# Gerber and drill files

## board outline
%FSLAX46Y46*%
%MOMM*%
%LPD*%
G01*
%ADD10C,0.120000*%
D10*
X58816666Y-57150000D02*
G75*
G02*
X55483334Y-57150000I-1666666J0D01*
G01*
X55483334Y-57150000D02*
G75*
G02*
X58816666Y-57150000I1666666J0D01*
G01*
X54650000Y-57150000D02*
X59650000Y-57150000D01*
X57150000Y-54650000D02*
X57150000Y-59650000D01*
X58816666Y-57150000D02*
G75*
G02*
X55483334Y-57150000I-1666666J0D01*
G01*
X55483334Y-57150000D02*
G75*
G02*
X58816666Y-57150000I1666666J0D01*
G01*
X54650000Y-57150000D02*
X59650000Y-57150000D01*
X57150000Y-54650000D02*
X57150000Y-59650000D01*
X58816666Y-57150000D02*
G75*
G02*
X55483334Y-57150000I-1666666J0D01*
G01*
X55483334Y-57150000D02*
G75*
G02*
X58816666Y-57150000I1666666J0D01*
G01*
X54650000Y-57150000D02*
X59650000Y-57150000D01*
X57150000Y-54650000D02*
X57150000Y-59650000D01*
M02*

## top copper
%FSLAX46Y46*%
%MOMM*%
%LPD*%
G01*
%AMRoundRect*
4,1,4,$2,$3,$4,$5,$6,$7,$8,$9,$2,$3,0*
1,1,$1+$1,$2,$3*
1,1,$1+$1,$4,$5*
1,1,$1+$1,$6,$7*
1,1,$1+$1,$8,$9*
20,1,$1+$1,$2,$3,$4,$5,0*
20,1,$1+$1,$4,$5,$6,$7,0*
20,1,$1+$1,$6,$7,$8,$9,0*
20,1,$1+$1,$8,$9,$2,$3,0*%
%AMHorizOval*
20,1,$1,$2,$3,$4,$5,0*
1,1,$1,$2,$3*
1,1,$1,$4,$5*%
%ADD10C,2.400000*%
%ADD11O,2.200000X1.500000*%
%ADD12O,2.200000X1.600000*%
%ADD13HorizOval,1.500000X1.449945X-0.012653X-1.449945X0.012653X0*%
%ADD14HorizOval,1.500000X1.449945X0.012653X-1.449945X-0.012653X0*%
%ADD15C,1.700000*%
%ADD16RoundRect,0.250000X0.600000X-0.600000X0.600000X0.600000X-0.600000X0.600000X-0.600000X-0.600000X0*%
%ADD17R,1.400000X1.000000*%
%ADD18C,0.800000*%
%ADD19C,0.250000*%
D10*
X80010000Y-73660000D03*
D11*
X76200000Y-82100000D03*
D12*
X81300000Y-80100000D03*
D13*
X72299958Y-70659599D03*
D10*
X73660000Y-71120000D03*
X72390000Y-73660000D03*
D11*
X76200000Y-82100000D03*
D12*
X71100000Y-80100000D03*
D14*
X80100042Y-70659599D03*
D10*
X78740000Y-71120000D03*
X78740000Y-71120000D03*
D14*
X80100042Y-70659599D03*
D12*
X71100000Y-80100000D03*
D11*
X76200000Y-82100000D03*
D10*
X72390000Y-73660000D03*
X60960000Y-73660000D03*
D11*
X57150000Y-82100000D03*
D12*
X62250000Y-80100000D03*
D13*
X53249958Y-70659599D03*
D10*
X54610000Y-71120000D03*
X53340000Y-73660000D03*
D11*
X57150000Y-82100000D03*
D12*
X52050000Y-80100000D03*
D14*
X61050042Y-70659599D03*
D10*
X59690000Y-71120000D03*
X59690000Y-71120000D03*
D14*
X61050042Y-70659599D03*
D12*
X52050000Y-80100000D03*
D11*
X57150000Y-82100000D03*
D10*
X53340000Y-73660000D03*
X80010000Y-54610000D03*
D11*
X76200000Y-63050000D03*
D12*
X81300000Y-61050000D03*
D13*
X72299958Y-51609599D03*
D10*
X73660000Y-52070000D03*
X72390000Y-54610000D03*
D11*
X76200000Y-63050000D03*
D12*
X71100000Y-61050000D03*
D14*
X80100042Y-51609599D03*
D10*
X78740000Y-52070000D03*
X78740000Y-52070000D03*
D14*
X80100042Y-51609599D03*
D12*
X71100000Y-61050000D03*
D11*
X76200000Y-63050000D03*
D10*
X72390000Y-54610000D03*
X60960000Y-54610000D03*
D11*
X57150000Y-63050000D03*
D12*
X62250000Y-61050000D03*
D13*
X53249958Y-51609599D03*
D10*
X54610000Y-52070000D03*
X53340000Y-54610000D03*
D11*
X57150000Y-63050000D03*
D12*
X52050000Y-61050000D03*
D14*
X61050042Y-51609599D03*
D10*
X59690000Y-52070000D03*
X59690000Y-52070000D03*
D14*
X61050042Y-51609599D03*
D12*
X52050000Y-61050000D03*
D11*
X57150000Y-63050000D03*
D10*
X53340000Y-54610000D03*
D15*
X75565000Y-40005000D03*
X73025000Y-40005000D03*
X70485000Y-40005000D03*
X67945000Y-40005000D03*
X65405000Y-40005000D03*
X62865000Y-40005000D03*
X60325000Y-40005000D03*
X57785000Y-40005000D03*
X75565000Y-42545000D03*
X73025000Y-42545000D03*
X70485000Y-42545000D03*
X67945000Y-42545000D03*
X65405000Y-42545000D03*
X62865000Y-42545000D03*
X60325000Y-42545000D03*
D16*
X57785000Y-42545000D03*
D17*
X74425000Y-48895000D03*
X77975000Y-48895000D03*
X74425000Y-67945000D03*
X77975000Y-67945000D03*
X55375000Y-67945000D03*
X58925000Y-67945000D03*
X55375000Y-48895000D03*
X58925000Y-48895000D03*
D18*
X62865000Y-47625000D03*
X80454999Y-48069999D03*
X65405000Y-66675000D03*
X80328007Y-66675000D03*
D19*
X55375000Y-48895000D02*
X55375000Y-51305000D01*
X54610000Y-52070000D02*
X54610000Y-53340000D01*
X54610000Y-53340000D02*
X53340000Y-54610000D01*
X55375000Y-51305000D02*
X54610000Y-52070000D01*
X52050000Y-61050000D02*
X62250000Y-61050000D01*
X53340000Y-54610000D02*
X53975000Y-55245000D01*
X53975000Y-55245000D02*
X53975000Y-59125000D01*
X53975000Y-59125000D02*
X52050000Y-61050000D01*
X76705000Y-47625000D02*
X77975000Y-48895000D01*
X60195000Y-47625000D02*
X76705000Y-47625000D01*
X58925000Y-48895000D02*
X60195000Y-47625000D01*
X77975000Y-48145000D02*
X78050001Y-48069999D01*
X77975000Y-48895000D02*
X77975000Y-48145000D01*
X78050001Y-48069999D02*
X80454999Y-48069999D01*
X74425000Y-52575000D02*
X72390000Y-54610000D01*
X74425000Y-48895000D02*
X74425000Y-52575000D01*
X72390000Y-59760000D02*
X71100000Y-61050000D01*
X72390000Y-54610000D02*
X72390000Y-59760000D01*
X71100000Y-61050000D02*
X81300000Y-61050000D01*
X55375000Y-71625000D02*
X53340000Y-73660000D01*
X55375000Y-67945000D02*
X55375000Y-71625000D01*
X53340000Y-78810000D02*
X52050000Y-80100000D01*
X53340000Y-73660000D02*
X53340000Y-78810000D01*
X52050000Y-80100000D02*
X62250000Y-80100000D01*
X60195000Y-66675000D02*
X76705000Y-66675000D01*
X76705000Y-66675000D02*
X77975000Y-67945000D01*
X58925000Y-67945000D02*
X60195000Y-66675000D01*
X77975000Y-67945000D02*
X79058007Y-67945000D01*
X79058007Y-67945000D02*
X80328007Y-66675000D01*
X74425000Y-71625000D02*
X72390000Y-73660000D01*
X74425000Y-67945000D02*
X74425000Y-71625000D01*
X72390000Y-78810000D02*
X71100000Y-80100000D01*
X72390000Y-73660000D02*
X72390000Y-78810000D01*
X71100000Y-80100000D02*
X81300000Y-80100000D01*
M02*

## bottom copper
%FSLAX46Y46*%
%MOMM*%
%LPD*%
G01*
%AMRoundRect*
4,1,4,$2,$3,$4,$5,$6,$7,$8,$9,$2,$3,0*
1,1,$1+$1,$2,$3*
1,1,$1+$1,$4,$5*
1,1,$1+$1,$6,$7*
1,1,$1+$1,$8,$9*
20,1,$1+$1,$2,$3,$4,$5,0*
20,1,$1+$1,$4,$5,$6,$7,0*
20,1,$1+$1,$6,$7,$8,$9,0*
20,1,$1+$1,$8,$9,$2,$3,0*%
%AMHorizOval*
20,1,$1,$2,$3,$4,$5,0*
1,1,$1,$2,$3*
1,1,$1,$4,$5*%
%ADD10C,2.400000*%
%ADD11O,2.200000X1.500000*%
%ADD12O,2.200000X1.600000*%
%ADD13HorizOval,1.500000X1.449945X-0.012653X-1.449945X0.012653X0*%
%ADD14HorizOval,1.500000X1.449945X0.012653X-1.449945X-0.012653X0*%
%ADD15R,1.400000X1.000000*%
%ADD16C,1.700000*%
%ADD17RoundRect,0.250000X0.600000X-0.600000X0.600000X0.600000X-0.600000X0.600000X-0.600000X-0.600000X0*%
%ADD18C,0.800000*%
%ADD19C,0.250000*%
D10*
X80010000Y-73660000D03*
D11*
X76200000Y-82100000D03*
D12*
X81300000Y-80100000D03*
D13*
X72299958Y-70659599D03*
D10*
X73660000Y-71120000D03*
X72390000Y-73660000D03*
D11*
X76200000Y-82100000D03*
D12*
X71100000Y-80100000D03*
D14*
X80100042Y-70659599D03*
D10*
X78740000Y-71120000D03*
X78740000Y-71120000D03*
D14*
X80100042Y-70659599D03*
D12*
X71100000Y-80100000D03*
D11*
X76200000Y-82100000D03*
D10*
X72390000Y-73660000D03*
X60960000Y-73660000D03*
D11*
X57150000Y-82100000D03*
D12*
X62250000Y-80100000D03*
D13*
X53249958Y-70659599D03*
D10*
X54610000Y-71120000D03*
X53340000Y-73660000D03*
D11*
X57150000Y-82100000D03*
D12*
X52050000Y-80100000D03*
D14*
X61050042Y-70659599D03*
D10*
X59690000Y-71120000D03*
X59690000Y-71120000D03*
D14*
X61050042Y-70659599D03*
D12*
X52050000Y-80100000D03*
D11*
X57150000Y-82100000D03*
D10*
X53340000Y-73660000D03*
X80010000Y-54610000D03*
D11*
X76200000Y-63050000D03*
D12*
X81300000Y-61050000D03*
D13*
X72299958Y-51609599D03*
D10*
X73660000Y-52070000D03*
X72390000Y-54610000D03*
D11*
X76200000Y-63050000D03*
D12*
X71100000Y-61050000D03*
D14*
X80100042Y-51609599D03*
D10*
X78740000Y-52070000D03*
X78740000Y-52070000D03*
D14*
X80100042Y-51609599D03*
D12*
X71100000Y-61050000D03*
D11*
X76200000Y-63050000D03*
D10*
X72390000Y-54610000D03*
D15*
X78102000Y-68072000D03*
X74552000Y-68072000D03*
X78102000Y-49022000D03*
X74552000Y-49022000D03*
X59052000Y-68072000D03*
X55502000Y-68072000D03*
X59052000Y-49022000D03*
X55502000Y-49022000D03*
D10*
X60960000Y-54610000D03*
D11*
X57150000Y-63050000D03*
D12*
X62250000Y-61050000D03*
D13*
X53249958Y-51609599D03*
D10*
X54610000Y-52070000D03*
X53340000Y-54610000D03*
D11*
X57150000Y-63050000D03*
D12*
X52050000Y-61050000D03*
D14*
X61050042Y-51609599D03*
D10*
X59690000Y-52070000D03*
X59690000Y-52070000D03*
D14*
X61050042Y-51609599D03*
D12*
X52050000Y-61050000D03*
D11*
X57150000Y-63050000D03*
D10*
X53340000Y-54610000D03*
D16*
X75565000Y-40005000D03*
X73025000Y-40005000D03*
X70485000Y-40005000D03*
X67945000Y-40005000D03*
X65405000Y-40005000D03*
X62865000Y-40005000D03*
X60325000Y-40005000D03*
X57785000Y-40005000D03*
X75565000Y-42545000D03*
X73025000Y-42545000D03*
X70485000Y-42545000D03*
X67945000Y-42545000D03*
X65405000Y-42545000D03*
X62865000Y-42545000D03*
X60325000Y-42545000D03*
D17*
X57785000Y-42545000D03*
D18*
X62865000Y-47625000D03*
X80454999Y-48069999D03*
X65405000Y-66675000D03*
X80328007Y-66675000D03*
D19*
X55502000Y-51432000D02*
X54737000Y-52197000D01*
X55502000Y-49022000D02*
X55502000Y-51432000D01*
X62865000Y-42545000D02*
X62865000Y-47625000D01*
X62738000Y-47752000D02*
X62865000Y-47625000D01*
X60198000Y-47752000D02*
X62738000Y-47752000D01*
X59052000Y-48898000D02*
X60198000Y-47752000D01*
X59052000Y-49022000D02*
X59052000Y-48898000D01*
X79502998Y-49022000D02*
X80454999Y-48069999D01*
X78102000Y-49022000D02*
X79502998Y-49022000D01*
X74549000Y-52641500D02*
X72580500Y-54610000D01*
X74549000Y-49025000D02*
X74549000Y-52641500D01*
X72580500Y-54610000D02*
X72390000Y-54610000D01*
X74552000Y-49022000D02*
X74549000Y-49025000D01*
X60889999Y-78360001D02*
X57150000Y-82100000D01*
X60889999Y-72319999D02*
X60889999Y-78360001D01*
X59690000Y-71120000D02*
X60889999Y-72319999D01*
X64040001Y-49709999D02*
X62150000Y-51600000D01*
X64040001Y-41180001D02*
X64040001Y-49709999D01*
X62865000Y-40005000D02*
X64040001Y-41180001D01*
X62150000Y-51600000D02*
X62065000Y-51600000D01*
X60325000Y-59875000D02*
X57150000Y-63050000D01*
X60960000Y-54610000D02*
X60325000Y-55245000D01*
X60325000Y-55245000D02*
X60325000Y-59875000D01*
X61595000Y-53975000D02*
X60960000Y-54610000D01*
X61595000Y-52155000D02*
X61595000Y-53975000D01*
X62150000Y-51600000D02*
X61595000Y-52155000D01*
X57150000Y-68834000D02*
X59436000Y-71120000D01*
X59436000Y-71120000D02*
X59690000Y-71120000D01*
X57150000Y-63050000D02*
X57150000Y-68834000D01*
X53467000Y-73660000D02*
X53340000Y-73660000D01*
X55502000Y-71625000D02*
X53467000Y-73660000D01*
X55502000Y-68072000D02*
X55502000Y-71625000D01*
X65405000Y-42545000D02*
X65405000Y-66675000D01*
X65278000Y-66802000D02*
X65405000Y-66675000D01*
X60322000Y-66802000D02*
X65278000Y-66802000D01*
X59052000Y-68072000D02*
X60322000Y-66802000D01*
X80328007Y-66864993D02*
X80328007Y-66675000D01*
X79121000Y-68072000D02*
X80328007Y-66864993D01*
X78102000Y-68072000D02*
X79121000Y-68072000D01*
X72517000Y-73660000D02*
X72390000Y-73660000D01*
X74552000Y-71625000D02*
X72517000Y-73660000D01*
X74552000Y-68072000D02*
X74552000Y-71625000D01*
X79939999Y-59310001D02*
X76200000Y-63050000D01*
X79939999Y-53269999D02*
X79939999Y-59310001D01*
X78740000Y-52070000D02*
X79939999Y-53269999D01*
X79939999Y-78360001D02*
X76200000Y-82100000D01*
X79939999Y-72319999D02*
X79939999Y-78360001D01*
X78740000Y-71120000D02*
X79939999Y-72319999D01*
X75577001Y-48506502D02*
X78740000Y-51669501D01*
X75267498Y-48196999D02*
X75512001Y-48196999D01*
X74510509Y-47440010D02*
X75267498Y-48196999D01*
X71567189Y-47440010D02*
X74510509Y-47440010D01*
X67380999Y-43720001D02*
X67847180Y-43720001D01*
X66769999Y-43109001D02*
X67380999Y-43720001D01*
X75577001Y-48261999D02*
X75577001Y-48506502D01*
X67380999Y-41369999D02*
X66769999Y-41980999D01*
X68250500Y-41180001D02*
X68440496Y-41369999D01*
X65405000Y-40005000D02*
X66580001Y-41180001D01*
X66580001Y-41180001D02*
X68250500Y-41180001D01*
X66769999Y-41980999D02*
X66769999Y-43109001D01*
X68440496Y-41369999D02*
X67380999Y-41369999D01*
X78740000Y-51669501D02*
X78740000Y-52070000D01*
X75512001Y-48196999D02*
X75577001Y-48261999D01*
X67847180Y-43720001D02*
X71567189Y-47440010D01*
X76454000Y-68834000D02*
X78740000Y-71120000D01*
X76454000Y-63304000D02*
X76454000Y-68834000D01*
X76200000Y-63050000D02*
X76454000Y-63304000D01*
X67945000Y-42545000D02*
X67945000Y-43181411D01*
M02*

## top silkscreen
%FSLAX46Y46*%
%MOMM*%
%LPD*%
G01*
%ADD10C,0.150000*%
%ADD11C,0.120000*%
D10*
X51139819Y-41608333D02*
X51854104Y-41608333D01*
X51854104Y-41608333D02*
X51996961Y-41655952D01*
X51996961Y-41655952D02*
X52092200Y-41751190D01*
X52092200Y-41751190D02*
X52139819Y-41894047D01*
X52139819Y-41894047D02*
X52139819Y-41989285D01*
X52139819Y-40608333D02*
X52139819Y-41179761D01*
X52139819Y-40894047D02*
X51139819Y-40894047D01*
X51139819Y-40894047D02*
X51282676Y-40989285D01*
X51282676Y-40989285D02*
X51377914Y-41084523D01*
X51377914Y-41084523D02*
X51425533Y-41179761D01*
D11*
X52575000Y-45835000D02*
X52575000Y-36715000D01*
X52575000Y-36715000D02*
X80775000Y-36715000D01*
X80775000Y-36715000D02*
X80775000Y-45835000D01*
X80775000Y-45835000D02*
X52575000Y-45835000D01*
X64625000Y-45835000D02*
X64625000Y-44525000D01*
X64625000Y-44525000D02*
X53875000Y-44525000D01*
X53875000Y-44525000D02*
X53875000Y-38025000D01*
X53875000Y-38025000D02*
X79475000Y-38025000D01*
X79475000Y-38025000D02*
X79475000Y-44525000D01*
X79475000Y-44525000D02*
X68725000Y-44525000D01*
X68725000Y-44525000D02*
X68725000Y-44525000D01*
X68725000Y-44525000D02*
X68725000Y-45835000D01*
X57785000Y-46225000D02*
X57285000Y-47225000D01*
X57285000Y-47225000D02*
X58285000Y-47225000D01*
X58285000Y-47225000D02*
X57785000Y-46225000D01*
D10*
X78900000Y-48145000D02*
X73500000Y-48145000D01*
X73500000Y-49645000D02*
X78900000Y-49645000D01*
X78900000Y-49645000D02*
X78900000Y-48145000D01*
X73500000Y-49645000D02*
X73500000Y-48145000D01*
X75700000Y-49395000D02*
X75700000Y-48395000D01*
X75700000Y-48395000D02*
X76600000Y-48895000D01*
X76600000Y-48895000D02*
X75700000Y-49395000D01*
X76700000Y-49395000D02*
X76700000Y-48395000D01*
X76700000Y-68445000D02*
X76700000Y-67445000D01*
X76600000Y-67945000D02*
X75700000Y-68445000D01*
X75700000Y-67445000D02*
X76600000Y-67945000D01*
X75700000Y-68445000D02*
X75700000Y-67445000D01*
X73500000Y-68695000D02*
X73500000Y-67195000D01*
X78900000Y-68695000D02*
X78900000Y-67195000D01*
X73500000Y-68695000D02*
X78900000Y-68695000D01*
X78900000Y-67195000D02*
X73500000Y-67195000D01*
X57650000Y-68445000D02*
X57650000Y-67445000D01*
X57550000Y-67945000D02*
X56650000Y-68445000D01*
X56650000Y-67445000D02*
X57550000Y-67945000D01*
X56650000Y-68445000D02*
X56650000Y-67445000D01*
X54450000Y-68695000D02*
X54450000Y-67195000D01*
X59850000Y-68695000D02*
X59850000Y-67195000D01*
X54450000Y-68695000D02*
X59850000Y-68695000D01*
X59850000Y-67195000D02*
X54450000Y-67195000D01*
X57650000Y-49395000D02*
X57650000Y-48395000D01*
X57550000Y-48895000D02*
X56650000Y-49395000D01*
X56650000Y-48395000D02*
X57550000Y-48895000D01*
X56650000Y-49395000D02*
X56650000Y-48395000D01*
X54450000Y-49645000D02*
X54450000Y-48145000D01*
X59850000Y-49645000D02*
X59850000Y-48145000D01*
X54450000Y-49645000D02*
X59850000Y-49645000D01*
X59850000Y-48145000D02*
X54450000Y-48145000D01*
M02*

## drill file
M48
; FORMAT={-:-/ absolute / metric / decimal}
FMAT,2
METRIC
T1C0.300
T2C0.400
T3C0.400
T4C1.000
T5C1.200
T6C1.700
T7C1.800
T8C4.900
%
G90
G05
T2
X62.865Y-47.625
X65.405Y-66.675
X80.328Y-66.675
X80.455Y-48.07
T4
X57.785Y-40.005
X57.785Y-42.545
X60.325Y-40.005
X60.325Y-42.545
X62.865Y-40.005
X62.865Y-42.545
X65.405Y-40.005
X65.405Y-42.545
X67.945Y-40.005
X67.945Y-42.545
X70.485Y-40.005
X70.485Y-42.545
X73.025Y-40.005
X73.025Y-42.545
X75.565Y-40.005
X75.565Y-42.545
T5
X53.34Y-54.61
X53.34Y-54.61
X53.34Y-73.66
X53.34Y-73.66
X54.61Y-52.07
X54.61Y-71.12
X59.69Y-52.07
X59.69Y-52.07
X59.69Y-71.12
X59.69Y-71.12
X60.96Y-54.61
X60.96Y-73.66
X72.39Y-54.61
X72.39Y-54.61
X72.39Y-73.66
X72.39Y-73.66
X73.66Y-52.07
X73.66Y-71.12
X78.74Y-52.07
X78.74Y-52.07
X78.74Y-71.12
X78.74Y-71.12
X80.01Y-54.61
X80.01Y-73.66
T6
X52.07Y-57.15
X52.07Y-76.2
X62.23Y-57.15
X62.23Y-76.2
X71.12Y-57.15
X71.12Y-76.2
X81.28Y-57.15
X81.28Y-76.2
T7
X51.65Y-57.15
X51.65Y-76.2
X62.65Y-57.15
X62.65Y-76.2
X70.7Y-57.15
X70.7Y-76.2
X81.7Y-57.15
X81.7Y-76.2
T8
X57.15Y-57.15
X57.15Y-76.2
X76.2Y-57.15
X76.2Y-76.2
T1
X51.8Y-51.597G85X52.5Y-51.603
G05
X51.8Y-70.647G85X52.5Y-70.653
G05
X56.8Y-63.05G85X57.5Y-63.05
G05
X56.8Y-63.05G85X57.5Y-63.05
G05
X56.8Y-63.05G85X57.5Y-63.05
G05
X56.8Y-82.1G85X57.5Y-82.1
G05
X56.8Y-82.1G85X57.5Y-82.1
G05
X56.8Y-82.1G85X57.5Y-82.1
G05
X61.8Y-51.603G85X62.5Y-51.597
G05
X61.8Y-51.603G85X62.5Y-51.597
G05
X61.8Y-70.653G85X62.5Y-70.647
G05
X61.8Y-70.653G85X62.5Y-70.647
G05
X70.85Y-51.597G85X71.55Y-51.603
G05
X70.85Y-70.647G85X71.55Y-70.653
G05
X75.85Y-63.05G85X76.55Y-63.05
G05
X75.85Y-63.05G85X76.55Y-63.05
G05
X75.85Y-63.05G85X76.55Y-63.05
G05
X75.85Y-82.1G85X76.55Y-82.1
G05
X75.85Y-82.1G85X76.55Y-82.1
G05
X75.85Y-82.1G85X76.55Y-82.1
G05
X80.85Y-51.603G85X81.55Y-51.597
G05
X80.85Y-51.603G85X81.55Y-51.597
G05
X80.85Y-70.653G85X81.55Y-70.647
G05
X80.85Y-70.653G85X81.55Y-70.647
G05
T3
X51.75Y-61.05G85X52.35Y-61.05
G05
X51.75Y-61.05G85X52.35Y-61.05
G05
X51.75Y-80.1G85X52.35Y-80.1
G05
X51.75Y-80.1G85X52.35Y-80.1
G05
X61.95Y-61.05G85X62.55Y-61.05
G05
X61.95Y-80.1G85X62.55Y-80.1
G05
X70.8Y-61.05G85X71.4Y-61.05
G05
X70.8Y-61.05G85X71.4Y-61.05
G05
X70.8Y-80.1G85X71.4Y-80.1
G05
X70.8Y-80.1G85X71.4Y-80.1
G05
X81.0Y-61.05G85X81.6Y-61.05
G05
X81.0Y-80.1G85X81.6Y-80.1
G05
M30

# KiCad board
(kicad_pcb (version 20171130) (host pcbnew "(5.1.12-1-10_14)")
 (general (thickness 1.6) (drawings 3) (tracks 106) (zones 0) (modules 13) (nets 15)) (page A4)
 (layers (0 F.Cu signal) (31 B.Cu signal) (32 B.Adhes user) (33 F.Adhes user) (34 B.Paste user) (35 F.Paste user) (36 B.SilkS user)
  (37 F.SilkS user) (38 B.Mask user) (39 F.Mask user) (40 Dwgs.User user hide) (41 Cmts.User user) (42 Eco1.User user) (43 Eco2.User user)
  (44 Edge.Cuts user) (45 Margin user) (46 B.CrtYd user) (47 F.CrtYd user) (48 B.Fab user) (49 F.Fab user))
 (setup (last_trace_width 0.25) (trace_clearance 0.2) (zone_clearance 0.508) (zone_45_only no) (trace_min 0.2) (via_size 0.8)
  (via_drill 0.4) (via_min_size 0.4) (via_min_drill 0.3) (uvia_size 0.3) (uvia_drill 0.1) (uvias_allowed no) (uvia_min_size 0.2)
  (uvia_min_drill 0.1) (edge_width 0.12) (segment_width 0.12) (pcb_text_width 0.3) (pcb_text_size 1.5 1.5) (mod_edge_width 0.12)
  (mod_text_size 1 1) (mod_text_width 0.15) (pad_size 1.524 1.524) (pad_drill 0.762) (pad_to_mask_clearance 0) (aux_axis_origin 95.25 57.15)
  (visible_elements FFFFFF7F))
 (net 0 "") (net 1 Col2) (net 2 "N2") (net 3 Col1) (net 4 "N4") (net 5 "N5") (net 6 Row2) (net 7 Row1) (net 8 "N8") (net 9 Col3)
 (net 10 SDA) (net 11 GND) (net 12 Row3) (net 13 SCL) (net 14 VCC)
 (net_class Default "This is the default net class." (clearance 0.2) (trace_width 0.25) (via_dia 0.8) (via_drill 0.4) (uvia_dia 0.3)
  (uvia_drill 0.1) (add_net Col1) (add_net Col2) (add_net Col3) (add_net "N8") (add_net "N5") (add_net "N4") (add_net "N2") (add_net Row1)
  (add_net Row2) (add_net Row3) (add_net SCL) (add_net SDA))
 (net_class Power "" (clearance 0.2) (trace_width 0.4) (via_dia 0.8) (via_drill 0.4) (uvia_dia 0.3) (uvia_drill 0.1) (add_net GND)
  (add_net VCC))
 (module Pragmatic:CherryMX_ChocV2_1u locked (layer F.Cu) (at 76.2 76.2)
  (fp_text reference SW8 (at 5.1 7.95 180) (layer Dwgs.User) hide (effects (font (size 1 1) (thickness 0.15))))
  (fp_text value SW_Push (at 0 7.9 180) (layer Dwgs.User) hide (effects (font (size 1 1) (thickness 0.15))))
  (pad 2 thru_hole circle (at 3.81 -2.54) (size 2.4 2.4) (drill 1.2) (layers *.Cu B.Mask) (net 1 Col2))
  (pad 2 thru_hole oval (at 0 5.9) (size 2.2 1.5) (drill oval 1 0.3) (layers *.Cu B.Mask) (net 1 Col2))
  (pad 1 thru_hole oval (at 5.1 3.9) (size 2.2 1.6) (drill oval 1 0.4) (layers *.Cu B.Mask) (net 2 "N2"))
  (pad 1 thru_hole oval (at -5 -5.55 359.5) (size 4.4 1.5) (drill oval 1 0.3 (offset 1.1 0)) (layers *.Cu B.Mask) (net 2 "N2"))
  (pad 1 thru_hole circle (at -2.54 -5.08) (size 2.4 2.4) (drill 1.2) (layers *.Cu B.Mask) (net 2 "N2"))
  (pad 1 thru_hole circle (at -3.81 -2.54) (size 2.4 2.4) (drill 1.2) (layers *.Cu B.Mask) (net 2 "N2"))
  (pad 2 thru_hole oval (at 0 5.9) (size 2.2 1.5) (drill oval 1 0.3) (layers *.Cu B.Mask) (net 1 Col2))
  (pad 1 thru_hole oval (at -5.1 3.9) (size 2.2 1.6) (drill oval 1 0.4) (layers *.Cu B.Mask) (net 2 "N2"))
  (pad 2 thru_hole oval (at 5 -5.55 0.5) (size 4.4 1.5) (drill oval 1 0.3 (offset -1.1 0)) (layers *.Cu B.Mask) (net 1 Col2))
  (pad 2 thru_hole circle (at 2.54 -5.08) (size 2.4 2.4) (drill 1.2) (layers *.Cu B.Mask) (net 1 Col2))
  (pad 2 thru_hole circle (at 2.54 -5.08) (size 2.4 2.4) (drill 1.2) (layers *.Cu B.Mask) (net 1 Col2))
  (pad 2 thru_hole oval (at 5 -5.55 0.5) (size 4.4 1.5) (drill oval 1 0.3 (offset -1.1 0)) (layers *.Cu B.Mask) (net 1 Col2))
  (pad 1 thru_hole oval (at -5.1 3.9) (size 2.2 1.6) (drill oval 1 0.4) (layers *.Cu B.Mask) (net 2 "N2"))
  (pad "" np_thru_hole circle (at 0 0 90) (size 4.9 4.9) (drill 4.9) (layers *.Cu *.Mask))
  (pad "" np_thru_hole circle (at -5.5 0 90) (size 1.8 1.8) (drill 1.8) (layers *.Cu *.Mask))
  (pad "" np_thru_hole circle (at 5.5 0 90) (size 1.8 1.8) (drill 1.8) (layers *.Cu *.Mask))
  (pad 2 thru_hole oval (at 0 5.9) (size 2.2 1.5) (drill oval 1 0.3) (layers *.Cu B.Mask) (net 1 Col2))
  (pad 1 thru_hole circle (at -3.81 -2.54) (size 2.4 2.4) (drill 1.2) (layers *.Cu B.Mask) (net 2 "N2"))
  (pad "" np_thru_hole circle (at 5.08 0) (size 1.7 1.7) (drill 1.7) (layers *.Cu *.Mask))
  (pad "" np_thru_hole circle (at -5.08 0) (size 1.7 1.7) (drill 1.7) (layers *.Cu *.Mask)))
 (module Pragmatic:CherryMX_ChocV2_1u (layer F.Cu) (at 57.15 76.2)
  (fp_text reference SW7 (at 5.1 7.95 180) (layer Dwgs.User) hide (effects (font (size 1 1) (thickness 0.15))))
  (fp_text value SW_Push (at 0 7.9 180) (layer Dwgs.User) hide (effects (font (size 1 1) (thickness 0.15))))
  (pad 2 thru_hole circle (at 3.81 -2.54) (size 2.4 2.4) (drill 1.2) (layers *.Cu B.Mask) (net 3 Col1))
  (pad 2 thru_hole oval (at 0 5.9) (size 2.2 1.5) (drill oval 1 0.3) (layers *.Cu B.Mask) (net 3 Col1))
  (pad 1 thru_hole oval (at 5.1 3.9) (size 2.2 1.6) (drill oval 1 0.4) (layers *.Cu B.Mask) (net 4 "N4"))
  (pad 1 thru_hole oval (at -5 -5.55 359.5) (size 4.4 1.5) (drill oval 1 0.3 (offset 1.1 0)) (layers *.Cu B.Mask) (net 4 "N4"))
  (pad 1 thru_hole circle (at -2.54 -5.08) (size 2.4 2.4) (drill 1.2) (layers *.Cu B.Mask) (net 4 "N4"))
  (pad 1 thru_hole circle (at -3.81 -2.54) (size 2.4 2.4) (drill 1.2) (layers *.Cu B.Mask) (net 4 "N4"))
  (pad 2 thru_hole oval (at 0 5.9) (size 2.2 1.5) (drill oval 1 0.3) (layers *.Cu B.Mask) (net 3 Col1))
  (pad 1 thru_hole oval (at -5.1 3.9) (size 2.2 1.6) (drill oval 1 0.4) (layers *.Cu B.Mask) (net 4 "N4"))
  (pad 2 thru_hole oval (at 5 -5.55 0.5) (size 4.4 1.5) (drill oval 1 0.3 (offset -1.1 0)) (layers *.Cu B.Mask) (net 3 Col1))
  (pad 2 thru_hole circle (at 2.54 -5.08) (size 2.4 2.4) (drill 1.2) (layers *.Cu B.Mask) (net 3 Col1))
  (pad 2 thru_hole circle (at 2.54 -5.08) (size 2.4 2.4) (drill 1.2) (layers *.Cu B.Mask) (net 3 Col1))
  (pad 2 thru_hole oval (at 5 -5.55 0.5) (size 4.4 1.5) (drill oval 1 0.3 (offset -1.1 0)) (layers *.Cu B.Mask) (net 3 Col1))
  (pad 1 thru_hole oval (at -5.1 3.9) (size 2.2 1.6) (drill oval 1 0.4) (layers *.Cu B.Mask) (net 4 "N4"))
  (pad "" np_thru_hole circle (at 0 0 90) (size 4.9 4.9) (drill 4.9) (layers *.Cu *.Mask))
  (pad "" np_thru_hole circle (at -5.5 0 90) (size 1.8 1.8) (drill 1.8) (layers *.Cu *.Mask))
  (pad "" np_thru_hole circle (at 5.5 0 90) (size 1.8 1.8) (drill 1.8) (layers *.Cu *.Mask))
  (pad 2 thru_hole oval (at 0 5.9) (size 2.2 1.5) (drill oval 1 0.3) (layers *.Cu B.Mask) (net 3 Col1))
  (pad 1 thru_hole circle (at -3.81 -2.54) (size 2.4 2.4) (drill 1.2) (layers *.Cu B.Mask) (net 4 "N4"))
  (pad "" np_thru_hole circle (at 5.08 0) (size 1.7 1.7) (drill 1.7) (layers *.Cu *.Mask))
  (pad "" np_thru_hole circle (at -5.08 0) (size 1.7 1.7) (drill 1.7) (layers *.Cu *.Mask)))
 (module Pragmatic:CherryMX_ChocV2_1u (layer F.Cu) (at 76.2 57.15)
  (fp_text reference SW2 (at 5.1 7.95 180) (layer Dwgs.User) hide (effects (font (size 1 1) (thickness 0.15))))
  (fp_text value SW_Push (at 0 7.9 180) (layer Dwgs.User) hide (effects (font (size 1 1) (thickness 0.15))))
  (pad 2 thru_hole circle (at 3.81 -2.54) (size 2.4 2.4) (drill 1.2) (layers *.Cu B.Mask) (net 1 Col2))
  (pad 2 thru_hole oval (at 0 5.9) (size 2.2 1.5) (drill oval 1 0.3) (layers *.Cu B.Mask) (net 1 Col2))
  (pad 1 thru_hole oval (at 5.1 3.9) (size 2.2 1.6) (drill oval 1 0.4) (layers *.Cu B.Mask) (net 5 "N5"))
  (pad 1 thru_hole oval (at -5 -5.55 359.5) (size 4.4 1.5) (drill oval 1 0.3 (offset 1.1 0)) (layers *.Cu B.Mask) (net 5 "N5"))
  (pad 1 thru_hole circle (at -2.54 -5.08) (size 2.4 2.4) (drill 1.2) (layers *.Cu B.Mask) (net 5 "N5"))
  (pad 1 thru_hole circle (at -3.81 -2.54) (size 2.4 2.4) (drill 1.2) (layers *.Cu B.Mask) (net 5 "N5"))
  (pad 2 thru_hole oval (at 0 5.9) (size 2.2 1.5) (drill oval 1 0.3) (layers *.Cu B.Mask) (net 1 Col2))
  (pad 1 thru_hole oval (at -5.1 3.9) (size 2.2 1.6) (drill oval 1 0.4) (layers *.Cu B.Mask) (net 5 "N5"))
  (pad 2 thru_hole oval (at 5 -5.55 0.5) (size 4.4 1.5) (drill oval 1 0.3 (offset -1.1 0)) (layers *.Cu B.Mask) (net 1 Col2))
  (pad 2 thru_hole circle (at 2.54 -5.08) (size 2.4 2.4) (drill 1.2) (layers *.Cu B.Mask) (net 1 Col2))
  (pad 2 thru_hole circle (at 2.54 -5.08) (size 2.4 2.4) (drill 1.2) (layers *.Cu B.Mask) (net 1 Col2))
  (pad 2 thru_hole oval (at 5 -5.55 0.5) (size 4.4 1.5) (drill oval 1 0.3 (offset -1.1 0)) (layers *.Cu B.Mask) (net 1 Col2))
  (pad 1 thru_hole oval (at -5.1 3.9) (size 2.2 1.6) (drill oval 1 0.4) (layers *.Cu B.Mask) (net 5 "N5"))
  (pad "" np_thru_hole circle (at 0 0 90) (size 4.9 4.9) (drill 4.9) (layers *.Cu *.Mask))
  (pad "" np_thru_hole circle (at -5.5 0 90) (size 1.8 1.8) (drill 1.8) (layers *.Cu *.Mask))
  (pad "" np_thru_hole circle (at 5.5 0 90) (size 1.8 1.8) (drill 1.8) (layers *.Cu *.Mask))
  (pad 2 thru_hole oval (at 0 5.9) (size 2.2 1.5) (drill oval 1 0.3) (layers *.Cu B.Mask) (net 1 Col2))
  (pad 1 thru_hole circle (at -3.81 -2.54) (size 2.4 2.4) (drill 1.2) (layers *.Cu B.Mask) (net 5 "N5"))
  (pad "" np_thru_hole circle (at 5.08 0) (size 1.7 1.7) (drill 1.7) (layers *.Cu *.Mask))
  (pad "" np_thru_hole circle (at -5.08 0) (size 1.7 1.7) (drill 1.7) (layers *.Cu *.Mask)))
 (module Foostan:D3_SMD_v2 (layer B.Cu) (at 76.327 68.072 180) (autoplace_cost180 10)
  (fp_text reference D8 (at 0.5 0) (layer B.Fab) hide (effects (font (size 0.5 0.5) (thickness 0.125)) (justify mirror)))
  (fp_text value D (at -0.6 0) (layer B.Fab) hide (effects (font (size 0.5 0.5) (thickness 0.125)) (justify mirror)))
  (pad 1 smd rect (at -1.775 0 180) (size 1.4 1) (layers B.Cu B.Paste B.Mask) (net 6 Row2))
  (pad 2 smd rect (at 1.775 0 180) (size 1.4 1) (layers B.Cu B.Paste B.Mask) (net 2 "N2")))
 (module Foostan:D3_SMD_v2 (layer B.Cu) (at 76.327 49.022 180) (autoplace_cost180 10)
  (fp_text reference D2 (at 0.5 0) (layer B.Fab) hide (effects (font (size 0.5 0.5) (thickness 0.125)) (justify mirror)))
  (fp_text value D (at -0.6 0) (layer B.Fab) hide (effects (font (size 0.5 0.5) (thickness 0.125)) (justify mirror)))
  (pad 1 smd rect (at -1.775 0 180) (size 1.4 1) (layers B.Cu B.Paste B.Mask) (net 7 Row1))
  (pad 2 smd rect (at 1.775 0 180) (size 1.4 1) (layers B.Cu B.Paste B.Mask) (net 5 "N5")))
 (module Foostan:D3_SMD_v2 (layer B.Cu) (at 57.277 68.072 180) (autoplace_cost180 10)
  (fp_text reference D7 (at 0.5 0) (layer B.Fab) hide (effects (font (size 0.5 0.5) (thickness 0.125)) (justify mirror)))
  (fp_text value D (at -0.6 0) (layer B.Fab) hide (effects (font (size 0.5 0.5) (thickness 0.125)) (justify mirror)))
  (pad 1 smd rect (at -1.775 0 180) (size 1.4 1) (layers B.Cu B.Paste B.Mask) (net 6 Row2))
  (pad 2 smd rect (at 1.775 0 180) (size 1.4 1) (layers B.Cu B.Paste B.Mask) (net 4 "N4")))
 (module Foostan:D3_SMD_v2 (layer B.Cu) (at 57.277 49.022 180) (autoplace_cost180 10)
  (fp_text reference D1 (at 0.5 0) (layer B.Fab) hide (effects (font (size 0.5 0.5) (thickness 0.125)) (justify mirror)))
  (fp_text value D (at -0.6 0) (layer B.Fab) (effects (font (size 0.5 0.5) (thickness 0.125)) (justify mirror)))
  (pad 1 smd rect (at -1.775 0 180) (size 1.4 1) (layers B.Cu B.Paste B.Mask) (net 7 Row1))
  (pad 2 smd rect (at 1.775 0 180) (size 1.4 1) (layers B.Cu B.Paste B.Mask) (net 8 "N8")))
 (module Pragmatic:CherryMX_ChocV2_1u (layer F.Cu) (at 57.15 57.15)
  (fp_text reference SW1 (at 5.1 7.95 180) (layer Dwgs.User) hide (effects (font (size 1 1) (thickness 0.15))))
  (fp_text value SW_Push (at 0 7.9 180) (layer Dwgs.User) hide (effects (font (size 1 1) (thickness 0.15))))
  (pad 2 thru_hole circle (at 3.81 -2.54) (size 2.4 2.4) (drill 1.2) (layers *.Cu B.Mask) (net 3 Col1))
  (pad 2 thru_hole oval (at 0 5.9) (size 2.2 1.5) (drill oval 1 0.3) (layers *.Cu B.Mask) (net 3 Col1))
  (pad 1 thru_hole oval (at 5.1 3.9) (size 2.2 1.6) (drill oval 1 0.4) (layers *.Cu B.Mask) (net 8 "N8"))
  (pad 1 thru_hole oval (at -5 -5.55 359.5) (size 4.4 1.5) (drill oval 1 0.3 (offset 1.1 0)) (layers *.Cu B.Mask) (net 8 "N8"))
  (pad 1 thru_hole circle (at -2.54 -5.08) (size 2.4 2.4) (drill 1.2) (layers *.Cu B.Mask) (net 8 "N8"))
  (pad 1 thru_hole circle (at -3.81 -2.54) (size 2.4 2.4) (drill 1.2) (layers *.Cu B.Mask) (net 8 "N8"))
  (pad 2 thru_hole oval (at 0 5.9) (size 2.2 1.5) (drill oval 1 0.3) (layers *.Cu B.Mask) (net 3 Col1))
  (pad 1 thru_hole oval (at -5.1 3.9) (size 2.2 1.6) (drill oval 1 0.4) (layers *.Cu B.Mask) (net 8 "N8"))
  (pad 2 thru_hole oval (at 5 -5.55 0.5) (size 4.4 1.5) (drill oval 1 0.3 (offset -1.1 0)) (layers *.Cu B.Mask) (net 3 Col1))
  (pad 2 thru_hole circle (at 2.54 -5.08) (size 2.4 2.4) (drill 1.2) (layers *.Cu B.Mask) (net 3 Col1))
  (pad 2 thru_hole circle (at 2.54 -5.08) (size 2.4 2.4) (drill 1.2) (layers *.Cu B.Mask) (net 3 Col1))
  (pad 2 thru_hole oval (at 5 -5.55 0.5) (size 4.4 1.5) (drill oval 1 0.3 (offset -1.1 0)) (layers *.Cu B.Mask) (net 3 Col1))
  (pad 1 thru_hole oval (at -5.1 3.9) (size 2.2 1.6) (drill oval 1 0.4) (layers *.Cu B.Mask) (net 8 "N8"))
  (pad "" np_thru_hole circle (at 0 0 90) (size 4.9 4.9) (drill 4.9) (layers *.Cu *.Mask))
  (pad "" np_thru_hole circle (at -5.5 0 90) (size 1.8 1.8) (drill 1.8) (layers *.Cu *.Mask))
  (pad "" np_thru_hole circle (at 5.5 0 90) (size 1.8 1.8) (drill 1.8) (layers *.Cu *.Mask))
  (pad 2 thru_hole oval (at 0 5.9) (size 2.2 1.5) (drill oval 1 0.3) (layers *.Cu B.Mask) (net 3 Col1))
  (pad 1 thru_hole circle (at -3.81 -2.54) (size 2.4 2.4) (drill 1.2) (layers *.Cu B.Mask) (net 8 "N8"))
  (pad "" np_thru_hole circle (at 5.08 0) (size 1.7 1.7) (drill 1.7) (layers *.Cu *.Mask))
  (pad "" np_thru_hole circle (at -5.08 0) (size 1.7 1.7) (drill 1.7) (layers *.Cu *.Mask)))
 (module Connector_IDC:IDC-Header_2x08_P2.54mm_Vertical (layer F.Cu) (at 57.785 42.545 90)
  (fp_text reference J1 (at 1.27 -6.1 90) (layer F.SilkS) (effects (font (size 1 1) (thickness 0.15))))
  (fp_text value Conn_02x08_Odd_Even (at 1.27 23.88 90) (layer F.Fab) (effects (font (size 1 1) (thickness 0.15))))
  (fp_line (start -3.29 -5.21) (end 5.83 -5.21) (layer F.SilkS) (width 0.12))
  (fp_line (start 5.83 -5.21) (end 5.83 22.99) (layer F.SilkS) (width 0.12))
  (fp_line (start 5.83 22.99) (end -3.29 22.99) (layer F.SilkS) (width 0.12))
  (fp_line (start -3.29 22.99) (end -3.29 -5.21) (layer F.SilkS) (width 0.12))
  (fp_line (start -3.29 6.84) (end -1.98 6.84) (layer F.SilkS) (width 0.12))
  (fp_line (start -1.98 6.84) (end -1.98 -3.91) (layer F.SilkS) (width 0.12))
  (fp_line (start -1.98 -3.91) (end 4.52 -3.91) (layer F.SilkS) (width 0.12))
  (fp_line (start 4.52 -3.91) (end 4.52 21.69) (layer F.SilkS) (width 0.12))
  (fp_line (start 4.52 21.69) (end -1.98 21.69) (layer F.SilkS) (width 0.12))
  (fp_line (start -1.98 21.69) (end -1.98 10.94) (layer F.SilkS) (width 0.12))
  (fp_line (start -1.98 10.94) (end -1.98 10.94) (layer F.SilkS) (width 0.12))
  (fp_line (start -1.98 10.94) (end -3.29 10.94) (layer F.SilkS) (width 0.12))
  (fp_line (start -3.68 0) (end -4.68 -0.5) (layer F.SilkS) (width 0.12))
  (fp_line (start -4.68 -0.5) (end -4.68 0.5) (layer F.SilkS) (width 0.12))
  (fp_line (start -4.68 0.5) (end -3.68 0) (layer F.SilkS) (width 0.12))
  (pad 16 thru_hole circle (at 2.54 17.78 90) (size 1.7 1.7) (drill 1) (layers *.Cu *.Mask))
  (pad 14 thru_hole circle (at 2.54 15.24 90) (size 1.7 1.7) (drill 1) (layers *.Cu *.Mask))
  (pad 12 thru_hole circle (at 2.54 12.7 90) (size 1.7 1.7) (drill 1) (layers *.Cu *.Mask))
  (pad 10 thru_hole circle (at 2.54 10.16 90) (size 1.7 1.7) (drill 1) (layers *.Cu *.Mask) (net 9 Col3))
  (pad 8 thru_hole circle (at 2.54 7.62 90) (size 1.7 1.7) (drill 1) (layers *.Cu *.Mask) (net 1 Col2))
  (pad 6 thru_hole circle (at 2.54 5.08 90) (size 1.7 1.7) (drill 1) (layers *.Cu *.Mask) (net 3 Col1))
  (pad 4 thru_hole circle (at 2.54 2.54 90) (size 1.7 1.7) (drill 1) (layers *.Cu *.Mask) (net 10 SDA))
  (pad 2 thru_hole circle (at 2.54 0 90) (size 1.7 1.7) (drill 1) (layers *.Cu *.Mask) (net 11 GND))
  (pad 15 thru_hole circle (at 0 17.78 90) (size 1.7 1.7) (drill 1) (layers *.Cu *.Mask))
  (pad 13 thru_hole circle (at 0 15.24 90) (size 1.7 1.7) (drill 1) (layers *.Cu *.Mask))
  (pad 11 thru_hole circle (at 0 12.7 90) (size 1.7 1.7) (drill 1) (layers *.Cu *.Mask))
  (pad 9 thru_hole circle (at 0 10.16 90) (size 1.7 1.7) (drill 1) (layers *.Cu *.Mask) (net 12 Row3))
  (pad 7 thru_hole circle (at 0 7.62 90) (size 1.7 1.7) (drill 1) (layers *.Cu *.Mask) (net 6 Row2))
  (pad 5 thru_hole circle (at 0 5.08 90) (size 1.7 1.7) (drill 1) (layers *.Cu *.Mask) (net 7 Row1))
  (pad 3 thru_hole circle (at 0 2.54 90) (size 1.7 1.7) (drill 1) (layers *.Cu *.Mask) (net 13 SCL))
  (pad 1 thru_hole roundrect (at 0 0 90) (size 1.7 1.7) (drill 1) (layers *.Cu *.Mask) (roundrect_rratio 0.147059) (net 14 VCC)))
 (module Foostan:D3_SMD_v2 (layer F.Cu) (at 76.2 48.895 180) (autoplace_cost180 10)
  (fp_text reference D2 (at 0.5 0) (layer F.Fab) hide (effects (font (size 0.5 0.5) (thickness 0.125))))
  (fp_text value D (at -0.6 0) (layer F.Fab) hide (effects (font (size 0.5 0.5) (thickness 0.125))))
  (fp_line (start -2.7 0.75) (end 2.7 0.75) (layer F.SilkS) (width 0.15))
  (fp_line (start 2.7 -0.75) (end -2.7 -0.75) (layer F.SilkS) (width 0.15))
  (fp_line (start -2.7 -0.75) (end -2.7 0.75) (layer F.SilkS) (width 0.15))
  (fp_line (start 2.7 -0.75) (end 2.7 0.75) (layer F.SilkS) (width 0.15))
  (fp_line (start 0.5 -0.5) (end 0.5 0.5) (layer F.SilkS) (width 0.15))
  (fp_line (start 0.5 0.5) (end -0.4 0) (layer F.SilkS) (width 0.15))
  (fp_line (start -0.4 0) (end 0.5 -0.5) (layer F.SilkS) (width 0.15))
  (fp_line (start -0.5 -0.5) (end -0.5 0.5) (layer F.SilkS) (width 0.15))
  (pad 2 smd rect (at 1.775 0 180) (size 1.4 1) (layers F.Cu F.Paste F.Mask) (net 5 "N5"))
  (pad 1 smd rect (at -1.775 0 180) (size 1.4 1) (layers F.Cu F.Paste F.Mask) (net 7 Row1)))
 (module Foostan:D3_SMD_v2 (layer F.Cu) (at 76.2 67.945 180) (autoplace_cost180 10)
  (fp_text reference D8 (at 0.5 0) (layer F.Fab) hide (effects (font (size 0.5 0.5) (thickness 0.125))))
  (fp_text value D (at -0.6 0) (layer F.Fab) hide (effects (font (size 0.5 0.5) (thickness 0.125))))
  (fp_line (start -0.5 -0.5) (end -0.5 0.5) (layer F.SilkS) (width 0.15))
  (fp_line (start -0.4 0) (end 0.5 -0.5) (layer F.SilkS) (width 0.15))
  (fp_line (start 0.5 0.5) (end -0.4 0) (layer F.SilkS) (width 0.15))
  (fp_line (start 0.5 -0.5) (end 0.5 0.5) (layer F.SilkS) (width 0.15))
  (fp_line (start 2.7 -0.75) (end 2.7 0.75) (layer F.SilkS) (width 0.15))
  (fp_line (start -2.7 -0.75) (end -2.7 0.75) (layer F.SilkS) (width 0.15))
  (fp_line (start 2.7 -0.75) (end -2.7 -0.75) (layer F.SilkS) (width 0.15))
  (fp_line (start -2.7 0.75) (end 2.7 0.75) (layer F.SilkS) (width 0.15))
  (pad 2 smd rect (at 1.775 0 180) (size 1.4 1) (layers F.Cu F.Paste F.Mask) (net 2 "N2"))
  (pad 1 smd rect (at -1.775 0 180) (size 1.4 1) (layers F.Cu F.Paste F.Mask) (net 6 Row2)))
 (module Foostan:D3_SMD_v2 (layer F.Cu) (at 57.15 67.945 180) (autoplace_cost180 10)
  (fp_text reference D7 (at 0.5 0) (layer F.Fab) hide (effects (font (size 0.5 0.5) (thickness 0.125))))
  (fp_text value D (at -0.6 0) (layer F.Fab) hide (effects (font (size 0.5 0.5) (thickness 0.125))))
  (fp_line (start -0.5 -0.5) (end -0.5 0.5) (layer F.SilkS) (width 0.15))
  (fp_line (start -0.4 0) (end 0.5 -0.5) (layer F.SilkS) (width 0.15))
  (fp_line (start 0.5 0.5) (end -0.4 0) (layer F.SilkS) (width 0.15))
  (fp_line (start 0.5 -0.5) (end 0.5 0.5) (layer F.SilkS) (width 0.15))
  (fp_line (start 2.7 -0.75) (end 2.7 0.75) (layer F.SilkS) (width 0.15))
  (fp_line (start -2.7 -0.75) (end -2.7 0.75) (layer F.SilkS) (width 0.15))
  (fp_line (start 2.7 -0.75) (end -2.7 -0.75) (layer F.SilkS) (width 0.15))
  (fp_line (start -2.7 0.75) (end 2.7 0.75) (layer F.SilkS) (width 0.15))
  (pad 2 smd rect (at 1.775 0 180) (size 1.4 1) (layers F.Cu F.Paste F.Mask) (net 4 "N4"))
  (pad 1 smd rect (at -1.775 0 180) (size 1.4 1) (layers F.Cu F.Paste F.Mask) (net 6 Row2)))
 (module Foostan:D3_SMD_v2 (layer F.Cu) (at 57.15 48.895 180) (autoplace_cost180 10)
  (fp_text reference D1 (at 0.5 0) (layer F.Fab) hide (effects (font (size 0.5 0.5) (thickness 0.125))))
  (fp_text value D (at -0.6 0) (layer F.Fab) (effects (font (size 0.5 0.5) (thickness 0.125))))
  (fp_line (start -0.5 -0.5) (end -0.5 0.5) (layer F.SilkS) (width 0.15))
  (fp_line (start -0.4 0) (end 0.5 -0.5) (layer F.SilkS) (width 0.15))
  (fp_line (start 0.5 0.5) (end -0.4 0) (layer F.SilkS) (width 0.15))
  (fp_line (start 0.5 -0.5) (end 0.5 0.5) (layer F.SilkS) (width 0.15))
  (fp_line (start 2.7 -0.75) (end 2.7 0.75) (layer F.SilkS) (width 0.15))
  (fp_line (start -2.7 -0.75) (end -2.7 0.75) (layer F.SilkS) (width 0.15))
  (fp_line (start 2.7 -0.75) (end -2.7 -0.75) (layer F.SilkS) (width 0.15))
  (fp_line (start -2.7 0.75) (end 2.7 0.75) (layer F.SilkS) (width 0.15))
  (pad 2 smd rect (at 1.775 0 180) (size 1.4 1) (layers F.Cu F.Paste F.Mask) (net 8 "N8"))
  (pad 1 smd rect (at -1.775 0 180) (size 1.4 1) (layers F.Cu F.Paste F.Mask) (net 7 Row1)))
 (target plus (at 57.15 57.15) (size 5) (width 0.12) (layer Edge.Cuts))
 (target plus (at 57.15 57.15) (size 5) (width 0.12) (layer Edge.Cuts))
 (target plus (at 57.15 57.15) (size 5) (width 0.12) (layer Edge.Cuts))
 (segment (start 55.375 48.895) (end 55.375 51.305) (width 0.25) (layer F.Cu) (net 8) (status 30))
 (segment (start 54.61 52.07) (end 54.61 53.34) (width 0.25) (layer F.Cu) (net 8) (status 10))
 (segment (start 54.61 53.34) (end 53.34 54.61) (width 0.25) (layer F.Cu) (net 8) (status 20))
 (segment (start 55.375 51.305) (end 54.61 52.07) (width 0.25) (layer F.Cu) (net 8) (status 30))
 (segment (start 52.05 61.05) (end 62.25 61.05) (width 0.25) (layer F.Cu) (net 8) (status 30))
 (segment (start 53.34 54.61) (end 53.975 55.245) (width 0.25) (layer F.Cu) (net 8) (status 30))
 (segment (start 53.975 55.245) (end 53.975 59.125) (width 0.25) (layer F.Cu) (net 8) (status 10))
 (segment (start 53.975 59.125) (end 52.05 61.05) (width 0.25) (layer F.Cu) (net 8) (status 20))
 (segment (start 55.502 51.432) (end 54.737 52.197) (width 0.25) (layer B.Cu) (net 8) (status 30))
 (segment (start 55.502 49.022) (end 55.502 51.432) (width 0.25) (layer B.Cu) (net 8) (status 30))
 (segment (start 76.705 47.625) (end 77.975 48.895) (width 0.25) (layer F.Cu) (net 7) (status 20))
 (segment (start 60.195 47.625) (end 76.705 47.625) (width 0.25) (layer F.Cu) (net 7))
 (segment (start 58.925 48.895) (end 60.195 47.625) (width 0.25) (layer F.Cu) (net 7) (status 10))
 (via (at 62.865 47.625) (size 0.8) (drill 0.4) (layers F.Cu B.Cu) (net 7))
 (segment (start 62.865 42.545) (end 62.865 47.625) (width 0.25) (layer B.Cu) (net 7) (status 10))
 (segment (start 77.975 48.145) (end 78.050001 48.069999) (width 0.25) (layer F.Cu) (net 7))
 (segment (start 77.975 48.895) (end 77.975 48.145) (width 0.25) (layer F.Cu) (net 7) (status 10))
 (segment (start 62.738 47.752) (end 62.865 47.625) (width 0.25) (layer B.Cu) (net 7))
 (segment (start 60.198 47.752) (end 62.738 47.752) (width 0.25) (layer B.Cu) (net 7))
 (segment (start 59.052 48.898) (end 60.198 47.752) (width 0.25) (layer B.Cu) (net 7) (status 10))
 (segment (start 59.052 49.022) (end 59.052 48.898) (width 0.25) (layer B.Cu) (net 7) (status 30))
 (segment (start 79.502998 49.022) (end 80.454999 48.069999) (width 0.25) (layer B.Cu) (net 7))
 (via (at 80.454999 48.069999) (size 0.8) (drill 0.4) (layers F.Cu B.Cu) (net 7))
 (segment (start 78.102 49.022) (end 79.502998 49.022) (width 0.25) (layer B.Cu) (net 7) (status 10))
 (segment (start 78.050001 48.069999) (end 80.454999 48.069999) (width 0.25) (layer F.Cu) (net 7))
 (segment (start 74.425 52.575) (end 72.39 54.61) (width 0.25) (layer F.Cu) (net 5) (status 30))
 (segment (start 74.425 48.895) (end 74.425 52.575) (width 0.25) (layer F.Cu) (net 5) (status 30))
 (segment (start 72.39 59.76) (end 71.1 61.05) (width 0.25) (layer F.Cu) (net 5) (status 20))
 (segment (start 72.39 54.61) (end 72.39 59.76) (width 0.25) (layer F.Cu) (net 5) (status 10))
 (segment (start 74.549 52.6415) (end 72.5805 54.61) (width 0.25) (layer B.Cu) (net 5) (status 30))
 (segment (start 74.549 49.025) (end 74.549 52.6415) (width 0.25) (layer B.Cu) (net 5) (status 30))
 (segment (start 72.5805 54.61) (end 72.39 54.61) (width 0.25) (layer B.Cu) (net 5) (status 30))
 (segment (start 74.552 49.022) (end 74.549 49.025) (width 0.25) (layer B.Cu) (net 5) (status 30))
 (segment (start 71.1 61.05) (end 81.3 61.05) (width 0.25) (layer F.Cu) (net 5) (status 30))
 (segment (start 60.889999 78.360001) (end 57.15 82.1) (width 0.25) (layer B.Cu) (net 3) (status 20))
 (segment (start 60.889999 72.319999) (end 60.889999 78.360001) (width 0.25) (layer B.Cu) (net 3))
 (segment (start 59.69 71.12) (end 60.889999 72.319999) (width 0.25) (layer B.Cu) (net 3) (status 10))
 (segment (start 64.040001 49.709999) (end 62.15 51.6) (width 0.25) (layer B.Cu) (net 3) (status 20))
 (segment (start 64.040001 41.180001) (end 64.040001 49.709999) (width 0.25) (layer B.Cu) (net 3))
 (segment (start 62.865 40.005) (end 64.040001 41.180001) (width 0.25) (layer B.Cu) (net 3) (status 10))
 (segment (start 62.15 51.6) (end 62.065 51.6) (width 0.25) (layer B.Cu) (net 3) (status 30))
 (segment (start 60.325 59.875) (end 57.15 63.05) (width 0.25) (layer B.Cu) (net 3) (status 20))
 (segment (start 60.96 54.61) (end 60.325 55.245) (width 0.25) (layer B.Cu) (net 3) (status 30))
 (segment (start 60.325 55.245) (end 60.325 59.875) (width 0.25) (layer B.Cu) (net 3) (status 10))
 (segment (start 61.595 53.975) (end 60.96 54.61) (width 0.25) (layer B.Cu) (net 3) (status 30))
 (segment (start 61.595 52.155) (end 61.595 53.975) (width 0.25) (layer B.Cu) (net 3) (status 30))
 (segment (start 62.15 51.6) (end 61.595 52.155) (width 0.25) (layer B.Cu) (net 3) (status 30))
 (segment (start 57.15 68.834) (end 59.436 71.12) (width 0.25) (layer B.Cu) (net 3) (status 20))
 (segment (start 59.436 71.12) (end 59.69 71.12) (width 0.25) (layer B.Cu) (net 3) (status 30))
 (segment (start 57.15 63.05) (end 57.15 68.834) (width 0.25) (layer B.Cu) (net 3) (status 10))
 (segment (start 55.375 71.625) (end 53.34 73.66) (width 0.25) (layer F.Cu) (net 4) (status 30))
 (segment (start 55.375 67.945) (end 55.375 71.625) (width 0.25) (layer F.Cu) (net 4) (status 30))
 (segment (start 53.34 78.81) (end 52.05 80.1) (width 0.25) (layer F.Cu) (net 4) (status 20))
 (segment (start 53.34 73.66) (end 53.34 78.81) (width 0.25) (layer F.Cu) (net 4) (status 10))
 (segment (start 53.467 73.66) (end 53.34 73.66) (width 0.25) (layer B.Cu) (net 4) (status 30))
 (segment (start 55.502 71.625) (end 53.467 73.66) (width 0.25) (layer B.Cu) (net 4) (status 30))
 (segment (start 55.502 68.072) (end 55.502 71.625) (width 0.25) (layer B.Cu) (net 4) (status 30))
 (segment (start 52.05 80.1) (end 62.25 80.1) (width 0.25) (layer F.Cu) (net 4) (status 30))
 (segment (start 60.195 66.675) (end 76.705 66.675) (width 0.25) (layer F.Cu) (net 6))
 (segment (start 76.705 66.675) (end 77.975 67.945) (width 0.25) (layer F.Cu) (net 6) (status 20))
 (segment (start 58.925 67.945) (end 60.195 66.675) (width 0.25) (layer F.Cu) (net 6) (status 10))
 (via (at 65.405 66.675) (size 0.8) (drill 0.4) (layers F.Cu B.Cu) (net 6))
 (segment (start 65.405 42.545) (end 65.405 66.675) (width 0.25) (layer B.Cu) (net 6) (status 10))
 (segment (start 65.278 66.802) (end 65.405 66.675) (width 0.25) (layer B.Cu) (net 6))
 (segment (start 60.322 66.802) (end 65.278 66.802) (width 0.25) (layer B.Cu) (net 6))
 (segment (start 59.052 68.072) (end 60.322 66.802) (width 0.25) (layer B.Cu) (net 6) (status 10))
 (segment (start 77.975 67.945) (end 79.058007 67.945) (width 0.25) (layer F.Cu) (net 6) (status 10))
 (segment (start 79.058007 67.945) (end 80.328007 66.675) (width 0.25) (layer F.Cu) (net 6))
 (via (at 80.328007 66.675) (size 0.8) (drill 0.4) (layers F.Cu B.Cu) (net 6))
 (segment (start 80.328007 66.864993) (end 80.328007 66.675) (width 0.25) (layer B.Cu) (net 6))
 (segment (start 79.121 68.072) (end 80.328007 66.864993) (width 0.25) (layer B.Cu) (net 6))
 (segment (start 78.102 68.072) (end 79.121 68.072) (width 0.25) (layer B.Cu) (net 6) (status 10))
 (segment (start 74.425 71.625) (end 72.39 73.66) (width 0.25) (layer F.Cu) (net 2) (status 30))
 (segment (start 74.425 67.945) (end 74.425 71.625) (width 0.25) (layer F.Cu) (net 2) (status 30))
 (segment (start 72.39 78.81) (end 71.1 80.1) (width 0.25) (layer F.Cu) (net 2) (status 20))
 (segment (start 72.39 73.66) (end 72.39 78.81) (width 0.25) (layer F.Cu) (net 2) (status 10))
 (segment (start 72.517 73.66) (end 72.39 73.66) (width 0.25) (layer B.Cu) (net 2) (status 30))
 (segment (start 74.552 71.625) (end 72.517 73.66) (width 0.25) (layer B.Cu) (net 2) (status 30))
 (segment (start 74.552 68.072) (end 74.552 71.625) (width 0.25) (layer B.Cu) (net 2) (status 30))
 (segment (start 71.1 80.1) (end 81.3 80.1) (width 0.25) (layer F.Cu) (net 2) (status 30))
 (segment (start 79.939999 59.310001) (end 76.2 63.05) (width 0.25) (layer B.Cu) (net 1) (status 20))
 (segment (start 79.939999 53.269999) (end 79.939999 59.310001) (width 0.25) (layer B.Cu) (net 1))
 (segment (start 78.74 52.07) (end 79.939999 53.269999) (width 0.25) (layer B.Cu) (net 1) (status 10))
 (segment (start 79.939999 78.360001) (end 76.2 82.1) (width 0.25) (layer B.Cu) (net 1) (status 20))
 (segment (start 79.939999 72.319999) (end 79.939999 78.360001) (width 0.25) (layer B.Cu) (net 1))
 (segment (start 78.74 71.12) (end 79.939999 72.319999) (width 0.25) (layer B.Cu) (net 1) (status 10))
 (segment (start 75.577001 48.506502) (end 78.74 51.669501) (width 0.25) (layer B.Cu) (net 1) (status 20))
 (segment (start 75.267498 48.196999) (end 75.512001 48.196999) (width 0.25) (layer B.Cu) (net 1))
 (segment (start 74.510509 47.44001) (end 75.267498 48.196999) (width 0.25) (layer B.Cu) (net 1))
 (segment (start 71.567189 47.44001) (end 74.510509 47.44001) (width 0.25) (layer B.Cu) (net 1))
 (segment (start 67.380999 43.720001) (end 67.84718 43.720001) (width 0.25) (layer B.Cu) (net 1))
 (segment (start 66.769999 43.109001) (end 67.380999 43.720001) (width 0.25) (layer B.Cu) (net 1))
 (segment (start 75.577001 48.261999) (end 75.577001 48.506502) (width 0.25) (layer B.Cu) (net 1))
 (segment (start 67.380999 41.369999) (end 66.769999 41.980999) (width 0.25) (layer B.Cu) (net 1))
 (segment (start 68.2505 41.180001) (end 68.440496 41.369999) (width 0.25) (layer B.Cu) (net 1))
 (segment (start 65.405 40.005) (end 66.580001 41.180001) (width 0.25) (layer B.Cu) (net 1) (status 10))
 (segment (start 66.580001 41.180001) (end 68.2505 41.180001) (width 0.25) (layer B.Cu) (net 1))
 (segment (start 66.769999 41.980999) (end 66.769999 43.109001) (width 0.25) (layer B.Cu) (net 1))
 (segment (start 68.440496 41.369999) (end 67.380999 41.369999) (width 0.25) (layer B.Cu) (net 1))
 (segment (start 78.74 51.669501) (end 78.74 52.07) (width 0.25) (layer B.Cu) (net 1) (status 30))
 (segment (start 75.512001 48.196999) (end 75.577001 48.261999) (width 0.25) (layer B.Cu) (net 1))
 (segment (start 67.84718 43.720001) (end 71.567189 47.44001) (width 0.25) (layer B.Cu) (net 1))
 (segment (start 76.454 68.834) (end 78.74 71.12) (width 0.25) (layer B.Cu) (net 1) (status 20))
 (segment (start 76.454 63.304) (end 76.454 68.834) (width 0.25) (layer B.Cu) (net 1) (status 10))
 (segment (start 76.2 63.05) (end 76.454 63.304) (width 0.25) (layer B.Cu) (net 1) (status 30))
 (segment (start 67.945 42.545) (end 67.945 43.181411) (width 0.25) (layer B.Cu) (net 12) (status 30)))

